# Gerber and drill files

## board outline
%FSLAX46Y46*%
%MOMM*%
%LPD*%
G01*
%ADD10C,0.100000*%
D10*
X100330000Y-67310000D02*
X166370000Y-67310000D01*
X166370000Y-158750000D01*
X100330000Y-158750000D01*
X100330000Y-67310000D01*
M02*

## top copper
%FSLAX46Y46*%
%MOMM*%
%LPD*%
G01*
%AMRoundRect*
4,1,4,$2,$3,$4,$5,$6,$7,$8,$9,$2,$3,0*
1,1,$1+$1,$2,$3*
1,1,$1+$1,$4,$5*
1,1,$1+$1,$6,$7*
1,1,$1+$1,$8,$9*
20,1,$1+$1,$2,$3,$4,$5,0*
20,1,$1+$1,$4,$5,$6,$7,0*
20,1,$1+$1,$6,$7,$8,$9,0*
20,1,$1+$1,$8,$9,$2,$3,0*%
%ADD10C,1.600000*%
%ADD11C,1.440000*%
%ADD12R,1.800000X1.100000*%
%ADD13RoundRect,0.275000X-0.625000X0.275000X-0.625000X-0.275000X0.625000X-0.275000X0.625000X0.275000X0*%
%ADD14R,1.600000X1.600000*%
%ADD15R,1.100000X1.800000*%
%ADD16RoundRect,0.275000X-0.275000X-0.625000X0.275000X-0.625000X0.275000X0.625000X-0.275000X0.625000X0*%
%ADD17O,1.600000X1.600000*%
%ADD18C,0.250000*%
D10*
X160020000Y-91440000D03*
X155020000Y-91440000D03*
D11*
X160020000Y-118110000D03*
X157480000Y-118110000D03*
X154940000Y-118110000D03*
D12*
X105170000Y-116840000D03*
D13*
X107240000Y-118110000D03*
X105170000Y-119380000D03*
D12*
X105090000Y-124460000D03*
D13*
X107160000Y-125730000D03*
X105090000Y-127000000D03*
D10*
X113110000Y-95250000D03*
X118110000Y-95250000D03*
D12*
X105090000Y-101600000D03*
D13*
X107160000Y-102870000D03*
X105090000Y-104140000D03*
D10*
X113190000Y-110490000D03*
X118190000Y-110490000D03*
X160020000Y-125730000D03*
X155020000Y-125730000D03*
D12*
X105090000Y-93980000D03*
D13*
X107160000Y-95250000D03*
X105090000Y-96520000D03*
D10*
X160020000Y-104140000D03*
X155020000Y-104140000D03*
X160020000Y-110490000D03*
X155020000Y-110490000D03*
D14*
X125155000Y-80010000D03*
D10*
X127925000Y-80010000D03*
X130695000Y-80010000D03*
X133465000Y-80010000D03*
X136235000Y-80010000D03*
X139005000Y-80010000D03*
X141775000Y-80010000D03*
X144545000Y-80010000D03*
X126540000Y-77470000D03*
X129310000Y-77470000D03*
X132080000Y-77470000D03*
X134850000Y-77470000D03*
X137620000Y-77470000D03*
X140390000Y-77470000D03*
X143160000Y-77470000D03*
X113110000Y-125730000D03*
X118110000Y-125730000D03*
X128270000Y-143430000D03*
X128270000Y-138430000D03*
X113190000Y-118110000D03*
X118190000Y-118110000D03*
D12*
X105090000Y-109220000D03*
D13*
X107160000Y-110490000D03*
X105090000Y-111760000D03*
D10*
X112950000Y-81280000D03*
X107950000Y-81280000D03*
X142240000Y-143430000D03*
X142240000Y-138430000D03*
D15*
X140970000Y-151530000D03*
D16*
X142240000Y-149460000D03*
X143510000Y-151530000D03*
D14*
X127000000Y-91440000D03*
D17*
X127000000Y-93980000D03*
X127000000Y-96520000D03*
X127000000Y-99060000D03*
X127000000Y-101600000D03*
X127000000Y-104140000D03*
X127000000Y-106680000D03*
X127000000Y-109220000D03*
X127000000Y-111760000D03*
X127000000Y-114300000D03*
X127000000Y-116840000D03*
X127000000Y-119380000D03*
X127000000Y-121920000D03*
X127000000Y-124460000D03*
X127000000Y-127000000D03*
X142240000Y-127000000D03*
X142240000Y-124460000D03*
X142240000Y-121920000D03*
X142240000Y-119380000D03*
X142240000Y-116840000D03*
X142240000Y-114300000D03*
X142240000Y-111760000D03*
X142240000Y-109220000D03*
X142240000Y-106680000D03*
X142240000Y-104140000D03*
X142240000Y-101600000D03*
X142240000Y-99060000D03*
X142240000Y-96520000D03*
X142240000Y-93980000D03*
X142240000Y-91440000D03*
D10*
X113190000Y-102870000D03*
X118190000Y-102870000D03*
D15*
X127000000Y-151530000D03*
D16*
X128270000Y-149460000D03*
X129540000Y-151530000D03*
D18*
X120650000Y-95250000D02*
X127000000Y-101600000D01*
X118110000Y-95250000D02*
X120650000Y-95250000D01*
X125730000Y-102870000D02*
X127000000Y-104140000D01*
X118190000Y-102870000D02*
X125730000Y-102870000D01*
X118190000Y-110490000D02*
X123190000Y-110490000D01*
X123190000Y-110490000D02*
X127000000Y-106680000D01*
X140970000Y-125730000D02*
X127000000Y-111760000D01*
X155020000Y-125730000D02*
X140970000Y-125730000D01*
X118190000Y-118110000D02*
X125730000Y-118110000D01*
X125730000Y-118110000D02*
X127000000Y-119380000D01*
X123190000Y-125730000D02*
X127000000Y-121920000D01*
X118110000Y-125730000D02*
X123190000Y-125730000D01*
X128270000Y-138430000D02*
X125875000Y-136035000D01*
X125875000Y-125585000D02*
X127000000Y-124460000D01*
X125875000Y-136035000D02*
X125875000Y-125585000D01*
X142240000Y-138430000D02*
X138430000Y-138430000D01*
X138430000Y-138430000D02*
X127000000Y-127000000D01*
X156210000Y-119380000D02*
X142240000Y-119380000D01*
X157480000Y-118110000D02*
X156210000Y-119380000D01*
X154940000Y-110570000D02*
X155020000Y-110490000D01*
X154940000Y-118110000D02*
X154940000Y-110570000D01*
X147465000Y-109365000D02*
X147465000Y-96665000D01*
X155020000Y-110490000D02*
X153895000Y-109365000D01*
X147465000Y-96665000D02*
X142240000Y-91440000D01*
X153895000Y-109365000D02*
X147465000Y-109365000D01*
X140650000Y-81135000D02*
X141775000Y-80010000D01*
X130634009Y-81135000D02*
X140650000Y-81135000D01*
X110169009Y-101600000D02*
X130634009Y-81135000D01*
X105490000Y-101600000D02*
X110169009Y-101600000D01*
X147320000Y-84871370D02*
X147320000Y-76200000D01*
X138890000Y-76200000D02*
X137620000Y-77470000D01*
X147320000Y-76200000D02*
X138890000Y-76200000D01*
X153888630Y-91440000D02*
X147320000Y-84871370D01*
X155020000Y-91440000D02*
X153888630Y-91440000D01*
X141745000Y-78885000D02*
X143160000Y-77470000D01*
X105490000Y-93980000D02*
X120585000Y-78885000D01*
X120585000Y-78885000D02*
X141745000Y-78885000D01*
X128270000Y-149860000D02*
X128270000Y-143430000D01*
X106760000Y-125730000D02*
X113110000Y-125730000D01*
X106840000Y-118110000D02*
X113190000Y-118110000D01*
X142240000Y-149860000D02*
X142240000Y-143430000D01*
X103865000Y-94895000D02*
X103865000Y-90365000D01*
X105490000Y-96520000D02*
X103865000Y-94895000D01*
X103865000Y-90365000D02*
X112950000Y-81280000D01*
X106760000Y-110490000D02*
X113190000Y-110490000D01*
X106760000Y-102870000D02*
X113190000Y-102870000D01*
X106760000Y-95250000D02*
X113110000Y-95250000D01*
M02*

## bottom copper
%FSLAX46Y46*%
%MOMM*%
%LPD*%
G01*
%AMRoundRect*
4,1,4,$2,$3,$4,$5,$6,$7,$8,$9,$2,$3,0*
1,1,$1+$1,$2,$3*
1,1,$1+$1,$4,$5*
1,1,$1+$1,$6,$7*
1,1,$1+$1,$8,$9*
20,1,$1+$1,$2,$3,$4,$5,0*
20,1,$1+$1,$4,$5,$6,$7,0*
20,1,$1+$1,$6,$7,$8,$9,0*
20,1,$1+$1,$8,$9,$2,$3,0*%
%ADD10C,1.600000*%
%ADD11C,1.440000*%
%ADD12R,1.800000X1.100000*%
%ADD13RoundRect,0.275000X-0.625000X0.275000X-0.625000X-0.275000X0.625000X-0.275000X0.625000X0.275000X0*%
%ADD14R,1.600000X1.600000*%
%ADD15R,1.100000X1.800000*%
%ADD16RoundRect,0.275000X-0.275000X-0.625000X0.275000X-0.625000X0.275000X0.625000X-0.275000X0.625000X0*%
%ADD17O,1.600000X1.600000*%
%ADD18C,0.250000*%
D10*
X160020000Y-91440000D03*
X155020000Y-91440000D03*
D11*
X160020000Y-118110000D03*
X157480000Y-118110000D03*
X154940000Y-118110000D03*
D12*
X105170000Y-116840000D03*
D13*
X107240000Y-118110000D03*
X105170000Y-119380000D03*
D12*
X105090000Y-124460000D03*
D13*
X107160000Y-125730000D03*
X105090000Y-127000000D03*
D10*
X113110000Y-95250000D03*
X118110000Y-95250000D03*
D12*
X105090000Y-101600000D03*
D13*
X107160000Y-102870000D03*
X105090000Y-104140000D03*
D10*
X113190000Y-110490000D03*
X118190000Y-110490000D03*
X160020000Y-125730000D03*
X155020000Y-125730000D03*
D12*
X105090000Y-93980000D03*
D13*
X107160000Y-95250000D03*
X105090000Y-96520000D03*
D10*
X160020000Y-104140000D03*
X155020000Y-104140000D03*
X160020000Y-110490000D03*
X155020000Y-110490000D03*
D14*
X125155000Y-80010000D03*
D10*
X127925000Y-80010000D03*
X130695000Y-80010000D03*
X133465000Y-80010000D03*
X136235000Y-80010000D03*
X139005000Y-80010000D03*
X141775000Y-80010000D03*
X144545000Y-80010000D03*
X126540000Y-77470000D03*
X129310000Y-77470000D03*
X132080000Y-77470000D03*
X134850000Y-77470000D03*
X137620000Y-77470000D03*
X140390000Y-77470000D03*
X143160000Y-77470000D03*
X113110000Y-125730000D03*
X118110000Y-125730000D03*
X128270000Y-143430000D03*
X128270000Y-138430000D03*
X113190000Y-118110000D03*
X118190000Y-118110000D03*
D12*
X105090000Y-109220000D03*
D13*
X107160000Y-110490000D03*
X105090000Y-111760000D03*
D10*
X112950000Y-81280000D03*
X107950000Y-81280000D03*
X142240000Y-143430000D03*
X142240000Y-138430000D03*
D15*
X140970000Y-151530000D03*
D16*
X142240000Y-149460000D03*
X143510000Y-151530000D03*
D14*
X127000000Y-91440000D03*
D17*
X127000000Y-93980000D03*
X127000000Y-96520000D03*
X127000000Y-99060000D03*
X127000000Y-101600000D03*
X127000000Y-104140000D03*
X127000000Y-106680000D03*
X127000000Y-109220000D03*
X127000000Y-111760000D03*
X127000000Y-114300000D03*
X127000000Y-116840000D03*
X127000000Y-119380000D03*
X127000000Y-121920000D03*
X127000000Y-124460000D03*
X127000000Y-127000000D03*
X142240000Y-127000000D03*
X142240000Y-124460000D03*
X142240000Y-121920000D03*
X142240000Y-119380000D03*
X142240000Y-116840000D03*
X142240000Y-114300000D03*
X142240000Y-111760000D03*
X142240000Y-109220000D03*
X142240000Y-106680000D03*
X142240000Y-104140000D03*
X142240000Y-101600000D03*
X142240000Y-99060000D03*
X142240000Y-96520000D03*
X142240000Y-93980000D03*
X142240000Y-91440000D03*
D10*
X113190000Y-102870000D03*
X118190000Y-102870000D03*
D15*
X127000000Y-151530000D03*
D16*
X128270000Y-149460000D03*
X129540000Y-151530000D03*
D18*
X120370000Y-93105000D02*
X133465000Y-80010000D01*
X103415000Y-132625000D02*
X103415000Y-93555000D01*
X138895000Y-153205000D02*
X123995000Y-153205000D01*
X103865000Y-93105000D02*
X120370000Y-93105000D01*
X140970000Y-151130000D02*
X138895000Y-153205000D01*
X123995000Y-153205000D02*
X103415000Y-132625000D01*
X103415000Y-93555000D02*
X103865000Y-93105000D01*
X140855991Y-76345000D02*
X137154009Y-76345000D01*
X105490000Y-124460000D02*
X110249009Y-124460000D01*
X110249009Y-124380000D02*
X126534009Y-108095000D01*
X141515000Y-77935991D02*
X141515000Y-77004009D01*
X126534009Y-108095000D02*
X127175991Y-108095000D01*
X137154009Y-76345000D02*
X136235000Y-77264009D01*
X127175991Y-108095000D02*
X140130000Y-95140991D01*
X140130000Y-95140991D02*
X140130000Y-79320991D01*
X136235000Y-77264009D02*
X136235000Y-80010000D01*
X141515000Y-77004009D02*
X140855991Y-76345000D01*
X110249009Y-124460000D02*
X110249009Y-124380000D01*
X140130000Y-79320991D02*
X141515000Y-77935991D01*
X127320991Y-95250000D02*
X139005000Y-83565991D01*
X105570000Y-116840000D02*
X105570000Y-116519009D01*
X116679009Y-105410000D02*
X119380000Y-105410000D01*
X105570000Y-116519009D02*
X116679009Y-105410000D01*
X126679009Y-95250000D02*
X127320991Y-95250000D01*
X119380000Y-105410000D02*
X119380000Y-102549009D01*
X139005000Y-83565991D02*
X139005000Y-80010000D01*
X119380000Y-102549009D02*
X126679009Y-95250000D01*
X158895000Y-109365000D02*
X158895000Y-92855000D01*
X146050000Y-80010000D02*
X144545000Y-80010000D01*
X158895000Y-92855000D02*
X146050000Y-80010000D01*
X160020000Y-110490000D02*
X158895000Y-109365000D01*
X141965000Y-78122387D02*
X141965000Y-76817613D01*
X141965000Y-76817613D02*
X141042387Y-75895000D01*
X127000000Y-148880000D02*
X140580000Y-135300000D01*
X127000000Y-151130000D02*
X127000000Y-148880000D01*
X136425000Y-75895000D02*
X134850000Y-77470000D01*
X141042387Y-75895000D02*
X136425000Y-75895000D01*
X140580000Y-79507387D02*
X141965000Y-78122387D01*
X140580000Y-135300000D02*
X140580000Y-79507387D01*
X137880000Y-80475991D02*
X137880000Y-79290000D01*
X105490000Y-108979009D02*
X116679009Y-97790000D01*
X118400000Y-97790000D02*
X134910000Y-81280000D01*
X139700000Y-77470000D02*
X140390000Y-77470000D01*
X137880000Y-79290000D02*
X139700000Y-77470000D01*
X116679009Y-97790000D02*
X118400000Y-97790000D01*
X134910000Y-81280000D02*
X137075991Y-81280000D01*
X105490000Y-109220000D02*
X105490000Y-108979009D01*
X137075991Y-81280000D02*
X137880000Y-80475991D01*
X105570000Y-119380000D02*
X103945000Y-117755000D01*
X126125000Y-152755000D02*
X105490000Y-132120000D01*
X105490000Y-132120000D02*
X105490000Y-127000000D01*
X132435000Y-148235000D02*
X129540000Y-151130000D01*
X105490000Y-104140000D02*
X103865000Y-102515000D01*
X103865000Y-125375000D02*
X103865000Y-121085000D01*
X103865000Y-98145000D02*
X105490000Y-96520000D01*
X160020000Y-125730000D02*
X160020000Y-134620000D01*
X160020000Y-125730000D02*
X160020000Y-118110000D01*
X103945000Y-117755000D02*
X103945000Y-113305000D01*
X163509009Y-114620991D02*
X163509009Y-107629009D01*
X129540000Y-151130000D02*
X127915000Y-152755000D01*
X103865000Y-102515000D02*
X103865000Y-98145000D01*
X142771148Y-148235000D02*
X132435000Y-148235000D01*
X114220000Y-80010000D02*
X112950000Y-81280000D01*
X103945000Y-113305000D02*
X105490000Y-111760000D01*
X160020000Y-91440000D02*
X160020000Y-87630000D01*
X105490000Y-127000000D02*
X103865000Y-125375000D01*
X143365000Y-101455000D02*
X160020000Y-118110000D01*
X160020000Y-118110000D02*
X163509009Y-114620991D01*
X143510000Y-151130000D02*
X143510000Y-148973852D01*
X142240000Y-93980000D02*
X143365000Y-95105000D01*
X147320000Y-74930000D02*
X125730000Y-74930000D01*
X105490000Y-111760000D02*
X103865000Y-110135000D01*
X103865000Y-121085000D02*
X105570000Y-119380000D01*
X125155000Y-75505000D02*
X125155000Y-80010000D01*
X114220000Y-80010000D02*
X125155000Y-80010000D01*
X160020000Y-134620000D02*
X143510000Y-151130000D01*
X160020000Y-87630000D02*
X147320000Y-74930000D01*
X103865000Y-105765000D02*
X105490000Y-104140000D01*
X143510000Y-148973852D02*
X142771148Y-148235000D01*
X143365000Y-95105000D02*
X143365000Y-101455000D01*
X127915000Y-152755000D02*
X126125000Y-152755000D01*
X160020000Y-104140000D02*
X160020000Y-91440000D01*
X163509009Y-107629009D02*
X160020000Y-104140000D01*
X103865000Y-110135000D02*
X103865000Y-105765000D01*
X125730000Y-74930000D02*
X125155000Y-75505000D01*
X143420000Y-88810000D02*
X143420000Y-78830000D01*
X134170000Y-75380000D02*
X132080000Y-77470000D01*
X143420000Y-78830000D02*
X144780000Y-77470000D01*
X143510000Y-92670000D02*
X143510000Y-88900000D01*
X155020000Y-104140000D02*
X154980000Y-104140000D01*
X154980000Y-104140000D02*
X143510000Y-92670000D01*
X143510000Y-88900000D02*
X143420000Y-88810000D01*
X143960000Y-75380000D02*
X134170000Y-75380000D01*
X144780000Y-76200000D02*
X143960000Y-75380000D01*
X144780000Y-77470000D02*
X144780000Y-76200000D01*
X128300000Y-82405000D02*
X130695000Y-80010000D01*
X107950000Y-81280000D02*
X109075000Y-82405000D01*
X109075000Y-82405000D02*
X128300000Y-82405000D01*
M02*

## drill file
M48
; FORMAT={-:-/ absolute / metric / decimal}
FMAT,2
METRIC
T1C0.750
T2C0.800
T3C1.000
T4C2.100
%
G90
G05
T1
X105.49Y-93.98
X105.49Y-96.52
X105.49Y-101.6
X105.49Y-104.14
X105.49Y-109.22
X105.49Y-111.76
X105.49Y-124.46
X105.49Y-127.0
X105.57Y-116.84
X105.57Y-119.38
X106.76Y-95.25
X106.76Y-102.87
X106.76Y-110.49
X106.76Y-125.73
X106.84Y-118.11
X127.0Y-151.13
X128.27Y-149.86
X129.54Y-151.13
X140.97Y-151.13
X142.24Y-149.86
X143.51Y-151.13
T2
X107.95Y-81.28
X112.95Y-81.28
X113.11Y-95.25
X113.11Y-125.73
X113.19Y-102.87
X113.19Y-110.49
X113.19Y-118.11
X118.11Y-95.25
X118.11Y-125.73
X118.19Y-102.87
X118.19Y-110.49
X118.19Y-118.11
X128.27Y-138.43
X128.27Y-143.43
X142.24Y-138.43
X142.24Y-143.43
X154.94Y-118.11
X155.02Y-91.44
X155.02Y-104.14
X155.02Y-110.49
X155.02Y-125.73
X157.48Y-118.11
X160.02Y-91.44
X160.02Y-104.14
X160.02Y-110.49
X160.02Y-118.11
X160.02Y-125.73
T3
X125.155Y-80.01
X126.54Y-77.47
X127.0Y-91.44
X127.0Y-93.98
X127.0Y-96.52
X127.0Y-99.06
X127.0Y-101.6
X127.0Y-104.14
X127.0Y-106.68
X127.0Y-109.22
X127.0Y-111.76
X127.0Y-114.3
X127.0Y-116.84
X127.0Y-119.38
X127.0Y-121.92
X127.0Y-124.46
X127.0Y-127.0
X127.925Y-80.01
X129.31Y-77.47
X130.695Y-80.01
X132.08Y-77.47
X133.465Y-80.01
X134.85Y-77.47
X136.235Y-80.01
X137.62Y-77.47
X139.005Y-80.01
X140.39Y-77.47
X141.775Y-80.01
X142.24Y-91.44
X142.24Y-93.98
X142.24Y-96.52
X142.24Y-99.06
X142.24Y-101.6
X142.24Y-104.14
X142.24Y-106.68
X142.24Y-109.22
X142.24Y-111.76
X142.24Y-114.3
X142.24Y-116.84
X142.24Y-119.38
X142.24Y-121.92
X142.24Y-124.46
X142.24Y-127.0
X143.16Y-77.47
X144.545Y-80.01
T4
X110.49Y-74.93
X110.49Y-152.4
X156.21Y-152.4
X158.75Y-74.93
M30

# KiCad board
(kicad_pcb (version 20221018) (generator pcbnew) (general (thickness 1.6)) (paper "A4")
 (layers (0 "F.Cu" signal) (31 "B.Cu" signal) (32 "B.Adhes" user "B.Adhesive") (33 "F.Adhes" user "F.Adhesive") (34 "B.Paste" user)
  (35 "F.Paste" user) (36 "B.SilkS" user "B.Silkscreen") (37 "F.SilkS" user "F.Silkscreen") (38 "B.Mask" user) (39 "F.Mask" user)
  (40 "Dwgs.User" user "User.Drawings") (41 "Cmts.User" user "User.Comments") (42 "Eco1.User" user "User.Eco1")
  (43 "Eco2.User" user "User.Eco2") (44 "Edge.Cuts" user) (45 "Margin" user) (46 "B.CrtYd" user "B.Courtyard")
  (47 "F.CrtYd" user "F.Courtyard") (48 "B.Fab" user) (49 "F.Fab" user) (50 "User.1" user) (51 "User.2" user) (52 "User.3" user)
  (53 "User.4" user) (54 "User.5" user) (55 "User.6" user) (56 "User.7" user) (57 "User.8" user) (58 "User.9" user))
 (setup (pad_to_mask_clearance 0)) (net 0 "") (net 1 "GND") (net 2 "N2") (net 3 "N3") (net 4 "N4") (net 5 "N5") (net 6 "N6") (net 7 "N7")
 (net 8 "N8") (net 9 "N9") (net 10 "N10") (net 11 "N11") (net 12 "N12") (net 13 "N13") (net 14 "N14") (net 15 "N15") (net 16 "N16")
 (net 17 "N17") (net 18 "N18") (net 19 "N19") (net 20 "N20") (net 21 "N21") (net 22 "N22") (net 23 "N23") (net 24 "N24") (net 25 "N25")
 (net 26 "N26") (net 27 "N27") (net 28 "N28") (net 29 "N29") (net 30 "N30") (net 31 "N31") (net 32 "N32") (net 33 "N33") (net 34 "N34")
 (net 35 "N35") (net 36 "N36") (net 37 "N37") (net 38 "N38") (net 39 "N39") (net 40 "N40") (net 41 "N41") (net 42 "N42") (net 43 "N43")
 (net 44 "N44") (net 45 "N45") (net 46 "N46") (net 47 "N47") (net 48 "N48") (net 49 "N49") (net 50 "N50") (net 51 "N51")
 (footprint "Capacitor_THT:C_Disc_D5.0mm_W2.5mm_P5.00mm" (layer "F.Cu") (at 160.02 91.44 180)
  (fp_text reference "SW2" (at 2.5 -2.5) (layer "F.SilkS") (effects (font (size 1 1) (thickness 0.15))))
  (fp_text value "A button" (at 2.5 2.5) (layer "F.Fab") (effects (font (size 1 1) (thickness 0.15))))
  (pad "1" thru_hole circle (at 0 0 180) (size 1.6 1.6) (drill 0.8) (layers "*.Cu" "*.Mask") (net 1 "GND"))
  (pad "2" thru_hole circle (at 5 0 180) (size 1.6 1.6) (drill 0.8) (layers "*.Cu" "*.Mask") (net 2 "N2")))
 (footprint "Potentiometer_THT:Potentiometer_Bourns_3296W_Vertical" (layer "F.Cu") (at 160.02 118.11)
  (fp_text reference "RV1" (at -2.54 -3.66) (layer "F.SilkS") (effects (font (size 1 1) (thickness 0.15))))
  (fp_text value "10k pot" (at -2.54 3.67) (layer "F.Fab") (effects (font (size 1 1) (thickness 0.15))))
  (pad "1" thru_hole circle (at 0 0) (size 1.44 1.44) (drill 0.8) (layers "*.Cu" "*.Mask") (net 1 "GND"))
  (pad "2" thru_hole circle (at -2.54 0) (size 1.44 1.44) (drill 0.8) (layers "*.Cu" "*.Mask") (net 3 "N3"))
  (pad "3" thru_hole circle (at -5.08 0) (size 1.44 1.44) (drill 0.8) (layers "*.Cu" "*.Mask") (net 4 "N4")))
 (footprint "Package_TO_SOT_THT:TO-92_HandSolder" (layer "F.Cu") (at 105.57 116.84 -90)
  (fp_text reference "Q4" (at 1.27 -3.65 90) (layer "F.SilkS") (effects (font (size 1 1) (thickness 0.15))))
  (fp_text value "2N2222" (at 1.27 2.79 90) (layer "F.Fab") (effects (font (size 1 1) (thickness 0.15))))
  (pad "1" thru_hole rect (at 0 0 270) (size 1.1 1.8) (drill 0.75 (offset 0 0.4)) (layers "*.Cu" "*.Mask") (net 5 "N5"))
  (pad "2" thru_hole roundrect (at 1.27 -1.27 270) (size 1.1 1.8) (drill 0.75 (offset 0 -0.4)) (layers "*.Cu" "*.Mask")
   (roundrect_rratio 0.25) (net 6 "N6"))
  (pad "3" thru_hole roundrect (at 2.54 0 270) (size 1.1 1.8) (drill 0.75 (offset 0 0.4)) (layers "*.Cu" "*.Mask") (roundrect_rratio 0.25)
   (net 1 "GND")))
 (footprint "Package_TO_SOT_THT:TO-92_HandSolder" (layer "F.Cu") (at 105.49 124.46 -90)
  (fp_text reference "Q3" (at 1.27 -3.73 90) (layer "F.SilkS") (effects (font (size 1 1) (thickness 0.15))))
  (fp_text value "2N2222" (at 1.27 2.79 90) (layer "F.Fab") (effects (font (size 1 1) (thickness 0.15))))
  (pad "1" thru_hole rect (at 0 0 270) (size 1.1 1.8) (drill 0.75 (offset 0 0.4)) (layers "*.Cu" "*.Mask") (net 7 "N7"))
  (pad "2" thru_hole roundrect (at 1.27 -1.27 270) (size 1.1 1.8) (drill 0.75 (offset 0 -0.4)) (layers "*.Cu" "*.Mask")
   (roundrect_rratio 0.25) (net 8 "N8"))
  (pad "3" thru_hole roundrect (at 2.54 0 270) (size 1.1 1.8) (drill 0.75 (offset 0 0.4)) (layers "*.Cu" "*.Mask") (roundrect_rratio 0.25)
   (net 1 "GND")))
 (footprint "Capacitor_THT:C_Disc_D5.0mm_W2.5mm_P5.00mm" (layer "F.Cu") (at 113.11 95.25)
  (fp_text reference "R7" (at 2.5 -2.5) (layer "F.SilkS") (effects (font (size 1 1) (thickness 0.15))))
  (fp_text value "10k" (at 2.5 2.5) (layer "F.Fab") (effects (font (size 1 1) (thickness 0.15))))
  (pad "1" thru_hole circle (at 0 0) (size 1.6 1.6) (drill 0.8) (layers "*.Cu" "*.Mask") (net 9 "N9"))
  (pad "2" thru_hole circle (at 5 0) (size 1.6 1.6) (drill 0.8) (layers "*.Cu" "*.Mask") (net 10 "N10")))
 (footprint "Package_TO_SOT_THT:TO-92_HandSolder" (layer "F.Cu") (at 105.49 101.6 -90)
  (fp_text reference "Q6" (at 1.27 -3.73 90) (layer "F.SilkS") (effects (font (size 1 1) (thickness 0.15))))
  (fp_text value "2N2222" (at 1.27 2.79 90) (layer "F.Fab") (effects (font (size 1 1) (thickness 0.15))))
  (pad "1" thru_hole rect (at 0 0 270) (size 1.1 1.8) (drill 0.75 (offset 0 0.4)) (layers "*.Cu" "*.Mask") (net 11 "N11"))
  (pad "2" thru_hole roundrect (at 1.27 -1.27 270) (size 1.1 1.8) (drill 0.75 (offset 0 -0.4)) (layers "*.Cu" "*.Mask")
   (roundrect_rratio 0.25) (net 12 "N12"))
  (pad "3" thru_hole roundrect (at 2.54 0 270) (size 1.1 1.8) (drill 0.75 (offset 0 0.4)) (layers "*.Cu" "*.Mask") (roundrect_rratio 0.25)
   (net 1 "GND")))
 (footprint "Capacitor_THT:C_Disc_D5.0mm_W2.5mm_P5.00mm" (layer "F.Cu") (at 113.19 110.49)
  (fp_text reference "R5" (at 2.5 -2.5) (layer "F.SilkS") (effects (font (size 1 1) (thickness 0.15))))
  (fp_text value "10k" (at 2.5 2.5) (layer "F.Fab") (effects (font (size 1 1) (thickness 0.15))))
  (pad "1" thru_hole circle (at 0 0) (size 1.6 1.6) (drill 0.8) (layers "*.Cu" "*.Mask") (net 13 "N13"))
  (pad "2" thru_hole circle (at 5 0) (size 1.6 1.6) (drill 0.8) (layers "*.Cu" "*.Mask") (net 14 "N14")))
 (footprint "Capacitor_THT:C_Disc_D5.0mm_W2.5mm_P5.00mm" (layer "F.Cu") (at 160.02 125.73 180)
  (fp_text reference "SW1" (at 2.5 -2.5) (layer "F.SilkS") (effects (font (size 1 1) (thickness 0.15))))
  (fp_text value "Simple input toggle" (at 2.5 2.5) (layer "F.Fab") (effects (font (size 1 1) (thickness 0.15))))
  (pad "1" thru_hole circle (at 0 0 180) (size 1.6 1.6) (drill 0.8) (layers "*.Cu" "*.Mask") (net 1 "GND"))
  (pad "2" thru_hole circle (at 5 0 180) (size 1.6 1.6) (drill 0.8) (layers "*.Cu" "*.Mask") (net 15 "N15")))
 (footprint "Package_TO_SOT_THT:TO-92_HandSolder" (layer "F.Cu") (at 105.49 93.98 -90)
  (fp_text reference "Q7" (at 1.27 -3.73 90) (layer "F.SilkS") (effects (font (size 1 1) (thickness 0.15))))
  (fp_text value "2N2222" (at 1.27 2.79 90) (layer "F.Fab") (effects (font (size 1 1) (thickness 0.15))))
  (pad "1" thru_hole rect (at 0 0 270) (size 1.1 1.8) (drill 0.75 (offset 0 0.4)) (layers "*.Cu" "*.Mask") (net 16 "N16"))
  (pad "2" thru_hole roundrect (at 1.27 -1.27 270) (size 1.1 1.8) (drill 0.75 (offset 0 -0.4)) (layers "*.Cu" "*.Mask")
   (roundrect_rratio 0.25) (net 9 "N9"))
  (pad "3" thru_hole roundrect (at 2.54 0 270) (size 1.1 1.8) (drill 0.75 (offset 0 0.4)) (layers "*.Cu" "*.Mask") (roundrect_rratio 0.25)
   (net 1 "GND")))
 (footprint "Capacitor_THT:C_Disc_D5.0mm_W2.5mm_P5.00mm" (layer "F.Cu") (at 160.02 104.14 180)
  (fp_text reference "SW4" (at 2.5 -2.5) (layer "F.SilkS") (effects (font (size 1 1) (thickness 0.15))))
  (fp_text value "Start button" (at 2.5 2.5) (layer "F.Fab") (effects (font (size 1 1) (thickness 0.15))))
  (pad "1" thru_hole circle (at 0 0 180) (size 1.6 1.6) (drill 0.8) (layers "*.Cu" "*.Mask") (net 1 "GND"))
  (pad "2" thru_hole circle (at 5 0 180) (size 1.6 1.6) (drill 0.8) (layers "*.Cu" "*.Mask") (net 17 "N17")))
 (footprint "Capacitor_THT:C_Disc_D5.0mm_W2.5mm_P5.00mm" (layer "F.Cu") (at 160.02 110.49 180)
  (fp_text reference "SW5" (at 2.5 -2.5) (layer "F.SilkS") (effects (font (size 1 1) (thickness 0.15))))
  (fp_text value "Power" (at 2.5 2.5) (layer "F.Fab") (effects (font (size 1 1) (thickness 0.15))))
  (pad "1" thru_hole circle (at 0 0 180) (size 1.6 1.6) (drill 0.8) (layers "*.Cu" "*.Mask") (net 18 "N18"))
  (pad "2" thru_hole circle (at 5 0 180) (size 1.6 1.6) (drill 0.8) (layers "*.Cu" "*.Mask") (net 4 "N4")))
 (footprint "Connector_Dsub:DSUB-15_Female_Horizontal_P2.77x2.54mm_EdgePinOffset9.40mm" (layer "F.Cu") (at 125.155 80.01 180)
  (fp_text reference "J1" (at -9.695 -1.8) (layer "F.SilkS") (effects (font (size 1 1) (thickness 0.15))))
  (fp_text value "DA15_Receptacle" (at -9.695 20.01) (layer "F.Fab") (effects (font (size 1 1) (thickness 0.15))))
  (pad "1" thru_hole rect (at 0 0 180) (size 1.6 1.6) (drill 1) (layers "*.Cu" "*.Mask") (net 1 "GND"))
  (pad "2" thru_hole circle (at -2.77 0 180) (size 1.6 1.6) (drill 1) (layers "*.Cu" "*.Mask") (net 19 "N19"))
  (pad "3" thru_hole circle (at -5.54 0 180) (size 1.6 1.6) (drill 1) (layers "*.Cu" "*.Mask") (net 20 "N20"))
  (pad "4" thru_hole circle (at -8.31 0 180) (size 1.6 1.6) (drill 1) (layers "*.Cu" "*.Mask") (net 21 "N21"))
  (pad "5" thru_hole circle (at -11.08 0 180) (size 1.6 1.6) (drill 1) (layers "*.Cu" "*.Mask") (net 7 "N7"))
  (pad "6" thru_hole circle (at -13.85 0 180) (size 1.6 1.6) (drill 1) (layers "*.Cu" "*.Mask") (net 5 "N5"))
  (pad "7" thru_hole circle (at -16.62 0 180) (size 1.6 1.6) (drill 1) (layers "*.Cu" "*.Mask") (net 11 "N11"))
  (pad "8" thru_hole circle (at -19.39 0 180) (size 1.6 1.6) (drill 1) (layers "*.Cu" "*.Mask") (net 18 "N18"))
  (pad "9" thru_hole circle (at -1.385 2.54 180) (size 1.6 1.6) (drill 1) (layers "*.Cu" "*.Mask") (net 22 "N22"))
  (pad "10" thru_hole circle (at -4.155 2.54 180) (size 1.6 1.6) (drill 1) (layers "*.Cu" "*.Mask") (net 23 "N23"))
  (pad "11" thru_hole circle (at -6.925 2.54 180) (size 1.6 1.6) (drill 1) (layers "*.Cu" "*.Mask") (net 17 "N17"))
  (pad "12" thru_hole circle (at -9.695 2.54 180) (size 1.6 1.6) (drill 1) (layers "*.Cu" "*.Mask") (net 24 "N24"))
  (pad "13" thru_hole circle (at -12.465 2.54 180) (size 1.6 1.6) (drill 1) (layers "*.Cu" "*.Mask") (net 2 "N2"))
  (pad "14" thru_hole circle (at -15.235 2.54 180) (size 1.6 1.6) (drill 1) (layers "*.Cu" "*.Mask") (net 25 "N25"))
  (pad "15" thru_hole circle (at -18.005 2.54 180) (size 1.6 1.6) (drill 1) (layers "*.Cu" "*.Mask") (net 16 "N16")))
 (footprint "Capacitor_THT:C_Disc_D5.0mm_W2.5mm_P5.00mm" (layer "F.Cu") (at 113.11 125.73)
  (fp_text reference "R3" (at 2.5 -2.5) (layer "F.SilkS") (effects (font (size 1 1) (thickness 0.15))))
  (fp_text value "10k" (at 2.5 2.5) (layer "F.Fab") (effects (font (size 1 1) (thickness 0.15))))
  (pad "1" thru_hole circle (at 0 0) (size 1.6 1.6) (drill 0.8) (layers "*.Cu" "*.Mask") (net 8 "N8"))
  (pad "2" thru_hole circle (at 5 0) (size 1.6 1.6) (drill 0.8) (layers "*.Cu" "*.Mask") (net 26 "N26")))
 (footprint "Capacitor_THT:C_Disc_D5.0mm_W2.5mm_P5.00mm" (layer "F.Cu") (at 128.27 143.43 90)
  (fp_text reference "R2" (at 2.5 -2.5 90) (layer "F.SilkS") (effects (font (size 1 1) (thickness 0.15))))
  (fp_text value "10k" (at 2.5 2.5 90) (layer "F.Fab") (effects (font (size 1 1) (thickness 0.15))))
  (pad "1" thru_hole circle (at 0 0 90) (size 1.6 1.6) (drill 0.8) (layers "*.Cu" "*.Mask") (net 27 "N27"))
  (pad "2" thru_hole circle (at 5 0 90) (size 1.6 1.6) (drill 0.8) (layers "*.Cu" "*.Mask") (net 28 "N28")))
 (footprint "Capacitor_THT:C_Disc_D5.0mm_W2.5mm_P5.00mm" (layer "F.Cu") (at 113.19 118.11)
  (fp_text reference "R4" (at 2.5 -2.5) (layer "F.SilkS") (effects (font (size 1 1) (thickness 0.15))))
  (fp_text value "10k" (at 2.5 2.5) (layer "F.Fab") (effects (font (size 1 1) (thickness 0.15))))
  (pad "1" thru_hole circle (at 0 0) (size 1.6 1.6) (drill 0.8) (layers "*.Cu" "*.Mask") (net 6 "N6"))
  (pad "2" thru_hole circle (at 5 0) (size 1.6 1.6) (drill 0.8) (layers "*.Cu" "*.Mask") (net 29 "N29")))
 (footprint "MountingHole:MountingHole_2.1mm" (layer "F.Cu") (at 156.21 152.4)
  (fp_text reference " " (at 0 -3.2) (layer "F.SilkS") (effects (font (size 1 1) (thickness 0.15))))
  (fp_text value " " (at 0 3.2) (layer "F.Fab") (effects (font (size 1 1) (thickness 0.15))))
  (pad "" np_thru_hole circle (at 0 0) (size 2.1 2.1) (drill 2.1) (layers "F&B.Cu" "*.Mask")))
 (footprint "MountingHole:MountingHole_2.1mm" (layer "F.Cu") (at 110.49 152.4)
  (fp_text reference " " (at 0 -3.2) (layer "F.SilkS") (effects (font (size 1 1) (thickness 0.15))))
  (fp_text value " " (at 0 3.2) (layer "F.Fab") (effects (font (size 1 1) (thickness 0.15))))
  (pad "" np_thru_hole circle (at 0 0) (size 2.1 2.1) (drill 2.1) (layers "F&B.Cu" "*.Mask")))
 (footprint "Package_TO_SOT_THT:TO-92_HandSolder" (layer "F.Cu") (at 105.49 109.22 -90)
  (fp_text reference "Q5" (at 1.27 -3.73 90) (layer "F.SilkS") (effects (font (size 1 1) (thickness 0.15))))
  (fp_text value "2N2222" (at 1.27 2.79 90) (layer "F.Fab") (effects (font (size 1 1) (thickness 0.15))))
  (pad "1" thru_hole rect (at 0 0 270) (size 1.1 1.8) (drill 0.75 (offset 0 0.4)) (layers "*.Cu" "*.Mask") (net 25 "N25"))
  (pad "2" thru_hole roundrect (at 1.27 -1.27 270) (size 1.1 1.8) (drill 0.75 (offset 0 -0.4)) (layers "*.Cu" "*.Mask")
   (roundrect_rratio 0.25) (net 13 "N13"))
  (pad "3" thru_hole roundrect (at 2.54 0 270) (size 1.1 1.8) (drill 0.75 (offset 0 0.4)) (layers "*.Cu" "*.Mask") (roundrect_rratio 0.25)
   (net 1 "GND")))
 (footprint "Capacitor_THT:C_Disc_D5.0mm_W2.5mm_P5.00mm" (layer "F.Cu") (at 112.95 81.28 180)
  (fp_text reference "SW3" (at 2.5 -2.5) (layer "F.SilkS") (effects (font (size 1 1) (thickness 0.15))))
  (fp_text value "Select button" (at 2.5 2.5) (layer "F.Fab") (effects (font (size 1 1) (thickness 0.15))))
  (pad "1" thru_hole circle (at 0 0 180) (size 1.6 1.6) (drill 0.8) (layers "*.Cu" "*.Mask") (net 1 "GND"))
  (pad "2" thru_hole circle (at 5 0 180) (size 1.6 1.6) (drill 0.8) (layers "*.Cu" "*.Mask") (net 20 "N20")))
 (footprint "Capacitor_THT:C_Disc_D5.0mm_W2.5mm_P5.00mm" (layer "F.Cu") (at 142.24 143.43 90)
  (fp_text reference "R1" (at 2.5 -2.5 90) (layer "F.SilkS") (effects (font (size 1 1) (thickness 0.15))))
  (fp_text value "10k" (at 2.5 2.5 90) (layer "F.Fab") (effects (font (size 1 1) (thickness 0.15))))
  (pad "1" thru_hole circle (at 0 0 90) (size 1.6 1.6) (drill 0.8) (layers "*.Cu" "*.Mask") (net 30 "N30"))
  (pad "2" thru_hole circle (at 5 0 90) (size 1.6 1.6) (drill 0.8) (layers "*.Cu" "*.Mask") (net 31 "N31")))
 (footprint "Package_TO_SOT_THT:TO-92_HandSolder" (layer "F.Cu") (at 140.97 151.13)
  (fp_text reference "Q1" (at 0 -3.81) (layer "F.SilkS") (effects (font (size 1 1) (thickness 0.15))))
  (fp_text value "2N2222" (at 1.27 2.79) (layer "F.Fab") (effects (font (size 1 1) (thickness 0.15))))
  (pad "1" thru_hole rect (at 0 0) (size 1.1 1.8) (drill 0.75 (offset 0 0.4)) (layers "*.Cu" "*.Mask") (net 21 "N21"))
  (pad "2" thru_hole roundrect (at 1.27 -1.27) (size 1.1 1.8) (drill 0.75 (offset 0 -0.4)) (layers "*.Cu" "*.Mask") (roundrect_rratio 0.25)
   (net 30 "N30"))
  (pad "3" thru_hole roundrect (at 2.54 0) (size 1.1 1.8) (drill 0.75 (offset 0 0.4)) (layers "*.Cu" "*.Mask") (roundrect_rratio 0.25)
   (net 1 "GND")))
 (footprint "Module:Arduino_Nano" (layer "F.Cu") (at 127 91.44)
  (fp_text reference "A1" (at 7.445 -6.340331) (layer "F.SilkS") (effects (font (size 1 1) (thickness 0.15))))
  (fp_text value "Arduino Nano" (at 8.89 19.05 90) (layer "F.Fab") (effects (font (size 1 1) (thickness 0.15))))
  (pad "1" thru_hole rect (at 0 0) (size 1.6 1.6) (drill 1) (layers "*.Cu" "*.Mask") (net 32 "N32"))
  (pad "2" thru_hole oval (at 0 2.54) (size 1.6 1.6) (drill 1) (layers "*.Cu" "*.Mask") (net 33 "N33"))
  (pad "3" thru_hole oval (at 0 5.08) (size 1.6 1.6) (drill 1) (layers "*.Cu" "*.Mask") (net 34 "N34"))
  (pad "4" thru_hole oval (at 0 7.62) (size 1.6 1.6) (drill 1) (layers "*.Cu" "*.Mask") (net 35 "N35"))
  (pad "5" thru_hole oval (at 0 10.16) (size 1.6 1.6) (drill 1) (layers "*.Cu" "*.Mask") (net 10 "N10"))
  (pad "6" thru_hole oval (at 0 12.7) (size 1.6 1.6) (drill 1) (layers "*.Cu" "*.Mask") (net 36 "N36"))
  (pad "7" thru_hole oval (at 0 15.24) (size 1.6 1.6) (drill 1) (layers "*.Cu" "*.Mask") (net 14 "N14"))
  (pad "8" thru_hole oval (at 0 17.78) (size 1.6 1.6) (drill 1) (layers "*.Cu" "*.Mask") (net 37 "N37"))
  (pad "9" thru_hole oval (at 0 20.32) (size 1.6 1.6) (drill 1) (layers "*.Cu" "*.Mask") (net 15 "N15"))
  (pad "10" thru_hole oval (at 0 22.86) (size 1.6 1.6) (drill 1) (layers "*.Cu" "*.Mask") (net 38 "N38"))
  (pad "11" thru_hole oval (at 0 25.4) (size 1.6 1.6) (drill 1) (layers "*.Cu" "*.Mask") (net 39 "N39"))
  (pad "12" thru_hole oval (at 0 27.94) (size 1.6 1.6) (drill 1) (layers "*.Cu" "*.Mask") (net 29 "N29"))
  (pad "13" thru_hole oval (at 0 30.48) (size 1.6 1.6) (drill 1) (layers "*.Cu" "*.Mask") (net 26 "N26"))
  (pad "14" thru_hole oval (at 0 33.02) (size 1.6 1.6) (drill 1) (layers "*.Cu" "*.Mask") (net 28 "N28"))
  (pad "15" thru_hole oval (at 0 35.56) (size 1.6 1.6) (drill 1) (layers "*.Cu" "*.Mask") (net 31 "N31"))
  (pad "16" thru_hole oval (at 15.24 35.56) (size 1.6 1.6) (drill 1) (layers "*.Cu" "*.Mask") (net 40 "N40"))
  (pad "17" thru_hole oval (at 15.24 33.02) (size 1.6 1.6) (drill 1) (layers "*.Cu" "*.Mask") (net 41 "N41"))
  (pad "18" thru_hole oval (at 15.24 30.48) (size 1.6 1.6) (drill 1) (layers "*.Cu" "*.Mask") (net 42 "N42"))
  (pad "19" thru_hole oval (at 15.24 27.94) (size 1.6 1.6) (drill 1) (layers "*.Cu" "*.Mask") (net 3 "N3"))
  (pad "20" thru_hole oval (at 15.24 25.4) (size 1.6 1.6) (drill 1) (layers "*.Cu" "*.Mask") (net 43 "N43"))
  (pad "21" thru_hole oval (at 15.24 22.86) (size 1.6 1.6) (drill 1) (layers "*.Cu" "*.Mask") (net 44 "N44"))
  (pad "22" thru_hole oval (at 15.24 20.32) (size 1.6 1.6) (drill 1) (layers "*.Cu" "*.Mask") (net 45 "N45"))
  (pad "23" thru_hole oval (at 15.24 17.78) (size 1.6 1.6) (drill 1) (layers "*.Cu" "*.Mask") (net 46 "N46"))
  (pad "24" thru_hole oval (at 15.24 15.24) (size 1.6 1.6) (drill 1) (layers "*.Cu" "*.Mask") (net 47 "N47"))
  (pad "25" thru_hole oval (at 15.24 12.7) (size 1.6 1.6) (drill 1) (layers "*.Cu" "*.Mask") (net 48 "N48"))
  (pad "26" thru_hole oval (at 15.24 10.16) (size 1.6 1.6) (drill 1) (layers "*.Cu" "*.Mask") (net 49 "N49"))
  (pad "27" thru_hole oval (at 15.24 7.62) (size 1.6 1.6) (drill 1) (layers "*.Cu" "*.Mask") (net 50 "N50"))
  (pad "28" thru_hole oval (at 15.24 5.08) (size 1.6 1.6) (drill 1) (layers "*.Cu" "*.Mask") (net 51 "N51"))
  (pad "29" thru_hole oval (at 15.24 2.54) (size 1.6 1.6) (drill 1) (layers "*.Cu" "*.Mask") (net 1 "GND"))
  (pad "30" thru_hole oval (at 15.24 0) (size 1.6 1.6) (drill 1) (layers "*.Cu" "*.Mask") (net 4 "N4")))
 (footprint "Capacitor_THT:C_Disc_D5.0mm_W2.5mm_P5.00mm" (layer "F.Cu") (at 113.19 102.87)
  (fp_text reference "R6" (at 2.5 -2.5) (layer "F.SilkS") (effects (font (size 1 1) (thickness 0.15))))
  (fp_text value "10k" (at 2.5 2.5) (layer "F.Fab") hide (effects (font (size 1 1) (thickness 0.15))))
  (pad "1" thru_hole circle (at 0 0) (size 1.6 1.6) (drill 0.8) (layers "*.Cu" "*.Mask") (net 12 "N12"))
  (pad "2" thru_hole circle (at 5 0) (size 1.6 1.6) (drill 0.8) (layers "*.Cu" "*.Mask") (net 36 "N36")))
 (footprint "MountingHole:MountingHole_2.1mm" (layer "F.Cu") (at 110.49 74.93)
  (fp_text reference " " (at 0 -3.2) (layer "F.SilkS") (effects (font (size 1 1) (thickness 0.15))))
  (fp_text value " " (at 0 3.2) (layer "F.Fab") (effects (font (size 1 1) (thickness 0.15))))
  (pad "" np_thru_hole circle (at 0 0) (size 2.1 2.1) (drill 2.1) (layers "*.Cu" "*.Mask")))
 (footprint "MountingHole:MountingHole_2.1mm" (layer "F.Cu") (at 158.75 74.93)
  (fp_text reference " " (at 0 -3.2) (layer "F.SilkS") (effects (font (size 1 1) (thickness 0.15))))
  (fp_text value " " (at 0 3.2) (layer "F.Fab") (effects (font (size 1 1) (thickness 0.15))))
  (pad "" np_thru_hole circle (at 0 0) (size 2.1 2.1) (drill 2.1) (layers "F&B.Cu" "*.Mask")))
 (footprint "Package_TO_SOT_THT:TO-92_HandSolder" (layer "F.Cu") (at 127 151.13)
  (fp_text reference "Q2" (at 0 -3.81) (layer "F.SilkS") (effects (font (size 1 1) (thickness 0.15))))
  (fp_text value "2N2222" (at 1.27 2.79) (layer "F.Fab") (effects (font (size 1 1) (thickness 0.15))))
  (pad "1" thru_hole rect (at 0 0) (size 1.1 1.8) (drill 0.75 (offset 0 0.4)) (layers "*.Cu" "*.Mask") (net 24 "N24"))
  (pad "2" thru_hole roundrect (at 1.27 -1.27) (size 1.1 1.8) (drill 0.75 (offset 0 -0.4)) (layers "*.Cu" "*.Mask") (roundrect_rratio 0.25)
   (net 27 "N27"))
  (pad "3" thru_hole roundrect (at 2.54 0) (size 1.1 1.8) (drill 0.75 (offset 0 0.4)) (layers "*.Cu" "*.Mask") (roundrect_rratio 0.25)
   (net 1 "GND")))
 (gr_rect (start 100.33 67.31) (end 166.37 158.75) (stroke (width 0.1) (type default)) (fill none) (layer "Edge.Cuts"))
 (segment (start 120.65 95.25) (end 127 101.6) (width 0.25) (layer "F.Cu") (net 10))
 (segment (start 118.11 95.25) (end 120.65 95.25) (width 0.25) (layer "F.Cu") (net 10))
 (segment (start 125.73 102.87) (end 127 104.14) (width 0.25) (layer "F.Cu") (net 36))
 (segment (start 118.19 102.87) (end 125.73 102.87) (width 0.25) (layer "F.Cu") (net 36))
 (segment (start 118.19 110.49) (end 123.19 110.49) (width 0.25) (layer "F.Cu") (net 14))
 (segment (start 123.19 110.49) (end 127 106.68) (width 0.25) (layer "F.Cu") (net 14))
 (segment (start 140.97 125.73) (end 127 111.76) (width 0.25) (layer "F.Cu") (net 15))
 (segment (start 155.02 125.73) (end 140.97 125.73) (width 0.25) (layer "F.Cu") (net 15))
 (segment (start 118.19 118.11) (end 125.73 118.11) (width 0.25) (layer "F.Cu") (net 29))
 (segment (start 125.73 118.11) (end 127 119.38) (width 0.25) (layer "F.Cu") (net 29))
 (segment (start 123.19 125.73) (end 127 121.92) (width 0.25) (layer "F.Cu") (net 26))
 (segment (start 118.11 125.73) (end 123.19 125.73) (width 0.25) (layer "F.Cu") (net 26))
 (segment (start 128.27 138.43) (end 125.875 136.035) (width 0.25) (layer "F.Cu") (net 28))
 (segment (start 125.875 125.585) (end 127 124.46) (width 0.25) (layer "F.Cu") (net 28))
 (segment (start 125.875 136.035) (end 125.875 125.585) (width 0.25) (layer "F.Cu") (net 28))
 (segment (start 142.24 138.43) (end 138.43 138.43) (width 0.25) (layer "F.Cu") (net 31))
 (segment (start 138.43 138.43) (end 127 127) (width 0.25) (layer "F.Cu") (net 31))
 (segment (start 156.21 119.38) (end 142.24 119.38) (width 0.25) (layer "F.Cu") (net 3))
 (segment (start 157.48 118.11) (end 156.21 119.38) (width 0.25) (layer "F.Cu") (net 3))
 (segment (start 154.94 110.57) (end 155.02 110.49) (width 0.25) (layer "F.Cu") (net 4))
 (segment (start 154.94 118.11) (end 154.94 110.57) (width 0.25) (layer "F.Cu") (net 4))
 (segment (start 147.465 109.365) (end 147.465 96.665) (width 0.25) (layer "F.Cu") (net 4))
 (segment (start 155.02 110.49) (end 153.895 109.365) (width 0.25) (layer "F.Cu") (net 4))
 (segment (start 147.465 96.665) (end 142.24 91.44) (width 0.25) (layer "F.Cu") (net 4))
 (segment (start 153.895 109.365) (end 147.465 109.365) (width 0.25) (layer "F.Cu") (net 4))
 (segment (start 120.37 93.105) (end 133.465 80.01) (width 0.25) (layer "B.Cu") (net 21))
 (segment (start 103.415 132.625) (end 103.415 93.555) (width 0.25) (layer "B.Cu") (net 21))
 (segment (start 138.895 153.205) (end 123.995 153.205) (width 0.25) (layer "B.Cu") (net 21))
 (segment (start 103.865 93.105) (end 120.37 93.105) (width 0.25) (layer "B.Cu") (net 21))
 (segment (start 140.97 151.13) (end 138.895 153.205) (width 0.25) (layer "B.Cu") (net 21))
 (segment (start 123.995 153.205) (end 103.415 132.625) (width 0.25) (layer "B.Cu") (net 21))
 (segment (start 103.415 93.555) (end 103.865 93.105) (width 0.25) (layer "B.Cu") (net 21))
 (segment (start 140.855991 76.345) (end 137.154009 76.345) (width 0.25) (layer "B.Cu") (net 7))
 (segment (start 105.49 124.46) (end 110.249009 124.46) (width 0.25) (layer "B.Cu") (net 7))
 (segment (start 110.249009 124.38) (end 126.534009 108.095) (width 0.25) (layer "B.Cu") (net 7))
 (segment (start 141.515 77.935991) (end 141.515 77.004009) (width 0.25) (layer "B.Cu") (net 7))
 (segment (start 126.534009 108.095) (end 127.175991 108.095) (width 0.25) (layer "B.Cu") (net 7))
 (segment (start 137.154009 76.345) (end 136.235 77.264009) (width 0.25) (layer "B.Cu") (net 7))
 (segment (start 127.175991 108.095) (end 140.13 95.140991) (width 0.25) (layer "B.Cu") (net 7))
 (segment (start 140.13 95.140991) (end 140.13 79.320991) (width 0.25) (layer "B.Cu") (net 7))
 (segment (start 136.235 77.264009) (end 136.235 80.01) (width 0.25) (layer "B.Cu") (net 7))
 (segment (start 141.515 77.004009) (end 140.855991 76.345) (width 0.25) (layer "B.Cu") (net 7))
 (segment (start 110.249009 124.46) (end 110.249009 124.38) (width 0.25) (layer "B.Cu") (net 7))
 (segment (start 140.13 79.320991) (end 141.515 77.935991) (width 0.25) (layer "B.Cu") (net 7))
 (segment (start 127.320991 95.25) (end 139.005 83.565991) (width 0.25) (layer "B.Cu") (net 5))
 (segment (start 105.57 116.84) (end 105.57 116.519009) (width 0.25) (layer "B.Cu") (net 5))
 (segment (start 116.679009 105.41) (end 119.38 105.41) (width 0.25) (layer "B.Cu") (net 5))
 (segment (start 105.57 116.519009) (end 116.679009 105.41) (width 0.25) (layer "B.Cu") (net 5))
 (segment (start 126.679009 95.25) (end 127.320991 95.25) (width 0.25) (layer "B.Cu") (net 5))
 (segment (start 119.38 105.41) (end 119.38 102.549009) (width 0.25) (layer "B.Cu") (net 5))
 (segment (start 139.005 83.565991) (end 139.005 80.01) (width 0.25) (layer "B.Cu") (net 5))
 (segment (start 119.38 102.549009) (end 126.679009 95.25) (width 0.25) (layer "B.Cu") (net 5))
 (segment (start 140.65 81.135) (end 141.775 80.01) (width 0.25) (layer "F.Cu") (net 11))
 (segment (start 130.634009 81.135) (end 140.65 81.135) (width 0.25) (layer "F.Cu") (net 11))
 (segment (start 110.169009 101.6) (end 130.634009 81.135) (width 0.25) (layer "F.Cu") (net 11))
 (segment (start 105.49 101.6) (end 110.169009 101.6) (width 0.25) (layer "F.Cu") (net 11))
 (segment (start 158.895 109.365) (end 158.895 92.855) (width 0.25) (layer "B.Cu") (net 18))
 (segment (start 146.05 80.01) (end 144.545 80.01) (width 0.25) (layer "B.Cu") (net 18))
 (segment (start 158.895 92.855) (end 146.05 80.01) (width 0.25) (layer "B.Cu") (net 18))
 (segment (start 160.02 110.49) (end 158.895 109.365) (width 0.25) (layer "B.Cu") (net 18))
 (segment (start 141.965 78.122387) (end 141.965 76.817613) (width 0.25) (layer "B.Cu") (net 24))
 (segment (start 141.965 76.817613) (end 141.042387 75.895) (width 0.25) (layer "B.Cu") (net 24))
 (segment (start 127 148.88) (end 140.58 135.3) (width 0.25) (layer "B.Cu") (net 24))
 (segment (start 127 151.13) (end 127 148.88) (width 0.25) (layer "B.Cu") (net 24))
 (segment (start 136.425 75.895) (end 134.85 77.47) (width 0.25) (layer "B.Cu") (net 24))
 (segment (start 141.042387 75.895) (end 136.425 75.895) (width 0.25) (layer "B.Cu") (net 24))
 (segment (start 140.58 79.507387) (end 141.965 78.122387) (width 0.25) (layer "B.Cu") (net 24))
 (segment (start 140.58 135.3) (end 140.58 79.507387) (width 0.25) (layer "B.Cu") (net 24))
 (segment (start 147.32 84.87137) (end 147.32 76.2) (width 0.25) (layer "F.Cu") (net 2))
 (segment (start 138.89 76.2) (end 137.62 77.47) (width 0.25) (layer "F.Cu") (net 2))
 (segment (start 147.32 76.2) (end 138.89 76.2) (width 0.25) (layer "F.Cu") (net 2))
 (segment (start 153.88863 91.44) (end 147.32 84.87137) (width 0.25) (layer "F.Cu") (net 2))
 (segment (start 155.02 91.44) (end 153.88863 91.44) (width 0.25) (layer "F.Cu") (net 2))
 (segment (start 137.88 80.475991) (end 137.88 79.29) (width 0.25) (layer "B.Cu") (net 25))
 (segment (start 105.49 108.979009) (end 116.679009 97.79) (width 0.25) (layer "B.Cu") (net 25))
 (segment (start 118.4 97.79) (end 134.91 81.28) (width 0.25) (layer "B.Cu") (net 25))
 (segment (start 139.7 77.47) (end 140.39 77.47) (width 0.25) (layer "B.Cu") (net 25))
 (segment (start 137.88 79.29) (end 139.7 77.47) (width 0.25) (layer "B.Cu") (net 25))
 (segment (start 116.679009 97.79) (end 118.4 97.79) (width 0.25) (layer "B.Cu") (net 25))
 (segment (start 134.91 81.28) (end 137.075991 81.28) (width 0.25) (layer "B.Cu") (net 25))
 (segment (start 105.49 109.22) (end 105.49 108.979009) (width 0.25) (layer "B.Cu") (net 25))
 (segment (start 137.075991 81.28) (end 137.88 80.475991) (width 0.25) (layer "B.Cu") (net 25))
 (segment (start 141.745 78.885) (end 143.16 77.47) (width 0.25) (layer "F.Cu") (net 16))
 (segment (start 105.49 93.98) (end 120.585 78.885) (width 0.25) (layer "F.Cu") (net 16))
 (segment (start 120.585 78.885) (end 141.745 78.885) (width 0.25) (layer "F.Cu") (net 16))
 (segment (start 128.27 149.86) (end 128.27 143.43) (width 0.25) (layer "F.Cu") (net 27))
 (segment (start 106.76 125.73) (end 113.11 125.73) (width 0.25) (layer "F.Cu") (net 8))
 (segment (start 106.84 118.11) (end 113.19 118.11) (width 0.25) (layer "F.Cu") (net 6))
 (segment (start 142.24 149.86) (end 142.24 143.43) (width 0.25) (layer "F.Cu") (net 30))
 (segment (start 103.865 94.895) (end 103.865 90.365) (width 0.25) (layer "F.Cu") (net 1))
 (segment (start 105.49 96.52) (end 103.865 94.895) (width 0.25) (layer "F.Cu") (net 1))
 (segment (start 103.865 90.365) (end 112.95 81.28) (width 0.25) (layer "F.Cu") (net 1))
 (segment (start 105.57 119.38) (end 103.945 117.755) (width 0.25) (layer "B.Cu") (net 1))
 (segment (start 126.125 152.755) (end 105.49 132.12) (width 0.25) (layer "B.Cu") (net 1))
 (segment (start 105.49 132.12) (end 105.49 127) (width 0.25) (layer "B.Cu") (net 1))
 (segment (start 132.435 148.235) (end 129.54 151.13) (width 0.25) (layer "B.Cu") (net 1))
 (segment (start 105.49 104.14) (end 103.865 102.515) (width 0.25) (layer "B.Cu") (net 1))
 (segment (start 103.865 125.375) (end 103.865 121.085) (width 0.25) (layer "B.Cu") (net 1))
 (segment (start 103.865 98.145) (end 105.49 96.52) (width 0.25) (layer "B.Cu") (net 1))
 (segment (start 160.02 125.73) (end 160.02 134.62) (width 0.25) (layer "B.Cu") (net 1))
 (segment (start 160.02 125.73) (end 160.02 118.11) (width 0.25) (layer "B.Cu") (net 1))
 (segment (start 103.945 117.755) (end 103.945 113.305) (width 0.25) (layer "B.Cu") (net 1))
 (segment (start 163.509009 114.620991) (end 163.509009 107.629009) (width 0.25) (layer "B.Cu") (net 1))
 (segment (start 129.54 151.13) (end 127.915 152.755) (width 0.25) (layer "B.Cu") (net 1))
 (segment (start 103.865 102.515) (end 103.865 98.145) (width 0.25) (layer "B.Cu") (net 1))
 (segment (start 142.771148 148.235) (end 132.435 148.235) (width 0.25) (layer "B.Cu") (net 1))
 (segment (start 114.22 80.01) (end 112.95 81.28) (width 0.25) (layer "B.Cu") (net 1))
 (segment (start 103.945 113.305) (end 105.49 111.76) (width 0.25) (layer "B.Cu") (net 1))
 (segment (start 160.02 91.44) (end 160.02 87.63) (width 0.25) (layer "B.Cu") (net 1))
 (segment (start 105.49 127) (end 103.865 125.375) (width 0.25) (layer "B.Cu") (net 1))
 (segment (start 143.365 101.455) (end 160.02 118.11) (width 0.25) (layer "B.Cu") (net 1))
 (segment (start 160.02 118.11) (end 163.509009 114.620991) (width 0.25) (layer "B.Cu") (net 1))
 (segment (start 143.51 151.13) (end 143.51 148.973852) (width 0.25) (layer "B.Cu") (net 1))
 (segment (start 142.24 93.98) (end 143.365 95.105) (width 0.25) (layer "B.Cu") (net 1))
 (segment (start 147.32 74.93) (end 125.73 74.93) (width 0.25) (layer "B.Cu") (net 1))
 (segment (start 105.49 111.76) (end 103.865 110.135) (width 0.25) (layer "B.Cu") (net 1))
 (segment (start 103.865 121.085) (end 105.57 119.38) (width 0.25) (layer "B.Cu") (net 1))
 (segment (start 125.155 75.505) (end 125.155 80.01) (width 0.25) (layer "B.Cu") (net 1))
 (segment (start 114.22 80.01) (end 125.155 80.01) (width 0.25) (layer "B.Cu") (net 1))
 (segment (start 160.02 134.62) (end 143.51 151.13) (width 0.25) (layer "B.Cu") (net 1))
 (segment (start 160.02 87.63) (end 147.32 74.93) (width 0.25) (layer "B.Cu") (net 1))
 (segment (start 103.865 105.765) (end 105.49 104.14) (width 0.25) (layer "B.Cu") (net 1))
 (segment (start 143.51 148.973852) (end 142.771148 148.235) (width 0.25) (layer "B.Cu") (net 1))
 (segment (start 143.365 95.105) (end 143.365 101.455) (width 0.25) (layer "B.Cu") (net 1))
 (segment (start 127.915 152.755) (end 126.125 152.755) (width 0.25) (layer "B.Cu") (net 1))
 (segment (start 160.02 104.14) (end 160.02 91.44) (width 0.25) (layer "B.Cu") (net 1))
 (segment (start 163.509009 107.629009) (end 160.02 104.14) (width 0.25) (layer "B.Cu") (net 1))
 (segment (start 103.865 110.135) (end 103.865 105.765) (width 0.25) (layer "B.Cu") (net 1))
 (segment (start 125.73 74.93) (end 125.155 75.505) (width 0.25) (layer "B.Cu") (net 1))
 (segment (start 106.76 110.49) (end 113.19 110.49) (width 0.25) (layer "F.Cu") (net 13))
 (segment (start 106.76 102.87) (end 113.19 102.87) (width 0.25) (layer "F.Cu") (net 12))
 (segment (start 106.76 95.25) (end 113.11 95.25) (width 0.25) (layer "F.Cu") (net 9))
 (segment (start 143.42 88.81) (end 143.42 78.83) (width 0.25) (layer "B.Cu") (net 17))
 (segment (start 134.17 75.38) (end 132.08 77.47) (width 0.25) (layer "B.Cu") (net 17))
 (segment (start 143.42 78.83) (end 144.78 77.47) (width 0.25) (layer "B.Cu") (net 17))
 (segment (start 143.51 92.67) (end 143.51 88.9) (width 0.25) (layer "B.Cu") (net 17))
 (segment (start 155.02 104.14) (end 154.98 104.14) (width 0.25) (layer "B.Cu") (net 17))
 (segment (start 154.98 104.14) (end 143.51 92.67) (width 0.25) (layer "B.Cu") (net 17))
 (segment (start 143.51 88.9) (end 143.42 88.81) (width 0.25) (layer "B.Cu") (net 17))
 (segment (start 143.96 75.38) (end 134.17 75.38) (width 0.25) (layer "B.Cu") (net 17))
 (segment (start 144.78 76.2) (end 143.96 75.38) (width 0.25) (layer "B.Cu") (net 17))
 (segment (start 144.78 77.47) (end 144.78 76.2) (width 0.25) (layer "B.Cu") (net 17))
 (segment (start 128.3 82.405) (end 130.695 80.01) (width 0.25) (layer "B.Cu") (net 20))
 (segment (start 107.95 81.28) (end 109.075 82.405) (width 0.25) (layer "B.Cu") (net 20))
 (segment (start 109.075 82.405) (end 128.3 82.405) (width 0.25) (layer "B.Cu") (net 20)))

